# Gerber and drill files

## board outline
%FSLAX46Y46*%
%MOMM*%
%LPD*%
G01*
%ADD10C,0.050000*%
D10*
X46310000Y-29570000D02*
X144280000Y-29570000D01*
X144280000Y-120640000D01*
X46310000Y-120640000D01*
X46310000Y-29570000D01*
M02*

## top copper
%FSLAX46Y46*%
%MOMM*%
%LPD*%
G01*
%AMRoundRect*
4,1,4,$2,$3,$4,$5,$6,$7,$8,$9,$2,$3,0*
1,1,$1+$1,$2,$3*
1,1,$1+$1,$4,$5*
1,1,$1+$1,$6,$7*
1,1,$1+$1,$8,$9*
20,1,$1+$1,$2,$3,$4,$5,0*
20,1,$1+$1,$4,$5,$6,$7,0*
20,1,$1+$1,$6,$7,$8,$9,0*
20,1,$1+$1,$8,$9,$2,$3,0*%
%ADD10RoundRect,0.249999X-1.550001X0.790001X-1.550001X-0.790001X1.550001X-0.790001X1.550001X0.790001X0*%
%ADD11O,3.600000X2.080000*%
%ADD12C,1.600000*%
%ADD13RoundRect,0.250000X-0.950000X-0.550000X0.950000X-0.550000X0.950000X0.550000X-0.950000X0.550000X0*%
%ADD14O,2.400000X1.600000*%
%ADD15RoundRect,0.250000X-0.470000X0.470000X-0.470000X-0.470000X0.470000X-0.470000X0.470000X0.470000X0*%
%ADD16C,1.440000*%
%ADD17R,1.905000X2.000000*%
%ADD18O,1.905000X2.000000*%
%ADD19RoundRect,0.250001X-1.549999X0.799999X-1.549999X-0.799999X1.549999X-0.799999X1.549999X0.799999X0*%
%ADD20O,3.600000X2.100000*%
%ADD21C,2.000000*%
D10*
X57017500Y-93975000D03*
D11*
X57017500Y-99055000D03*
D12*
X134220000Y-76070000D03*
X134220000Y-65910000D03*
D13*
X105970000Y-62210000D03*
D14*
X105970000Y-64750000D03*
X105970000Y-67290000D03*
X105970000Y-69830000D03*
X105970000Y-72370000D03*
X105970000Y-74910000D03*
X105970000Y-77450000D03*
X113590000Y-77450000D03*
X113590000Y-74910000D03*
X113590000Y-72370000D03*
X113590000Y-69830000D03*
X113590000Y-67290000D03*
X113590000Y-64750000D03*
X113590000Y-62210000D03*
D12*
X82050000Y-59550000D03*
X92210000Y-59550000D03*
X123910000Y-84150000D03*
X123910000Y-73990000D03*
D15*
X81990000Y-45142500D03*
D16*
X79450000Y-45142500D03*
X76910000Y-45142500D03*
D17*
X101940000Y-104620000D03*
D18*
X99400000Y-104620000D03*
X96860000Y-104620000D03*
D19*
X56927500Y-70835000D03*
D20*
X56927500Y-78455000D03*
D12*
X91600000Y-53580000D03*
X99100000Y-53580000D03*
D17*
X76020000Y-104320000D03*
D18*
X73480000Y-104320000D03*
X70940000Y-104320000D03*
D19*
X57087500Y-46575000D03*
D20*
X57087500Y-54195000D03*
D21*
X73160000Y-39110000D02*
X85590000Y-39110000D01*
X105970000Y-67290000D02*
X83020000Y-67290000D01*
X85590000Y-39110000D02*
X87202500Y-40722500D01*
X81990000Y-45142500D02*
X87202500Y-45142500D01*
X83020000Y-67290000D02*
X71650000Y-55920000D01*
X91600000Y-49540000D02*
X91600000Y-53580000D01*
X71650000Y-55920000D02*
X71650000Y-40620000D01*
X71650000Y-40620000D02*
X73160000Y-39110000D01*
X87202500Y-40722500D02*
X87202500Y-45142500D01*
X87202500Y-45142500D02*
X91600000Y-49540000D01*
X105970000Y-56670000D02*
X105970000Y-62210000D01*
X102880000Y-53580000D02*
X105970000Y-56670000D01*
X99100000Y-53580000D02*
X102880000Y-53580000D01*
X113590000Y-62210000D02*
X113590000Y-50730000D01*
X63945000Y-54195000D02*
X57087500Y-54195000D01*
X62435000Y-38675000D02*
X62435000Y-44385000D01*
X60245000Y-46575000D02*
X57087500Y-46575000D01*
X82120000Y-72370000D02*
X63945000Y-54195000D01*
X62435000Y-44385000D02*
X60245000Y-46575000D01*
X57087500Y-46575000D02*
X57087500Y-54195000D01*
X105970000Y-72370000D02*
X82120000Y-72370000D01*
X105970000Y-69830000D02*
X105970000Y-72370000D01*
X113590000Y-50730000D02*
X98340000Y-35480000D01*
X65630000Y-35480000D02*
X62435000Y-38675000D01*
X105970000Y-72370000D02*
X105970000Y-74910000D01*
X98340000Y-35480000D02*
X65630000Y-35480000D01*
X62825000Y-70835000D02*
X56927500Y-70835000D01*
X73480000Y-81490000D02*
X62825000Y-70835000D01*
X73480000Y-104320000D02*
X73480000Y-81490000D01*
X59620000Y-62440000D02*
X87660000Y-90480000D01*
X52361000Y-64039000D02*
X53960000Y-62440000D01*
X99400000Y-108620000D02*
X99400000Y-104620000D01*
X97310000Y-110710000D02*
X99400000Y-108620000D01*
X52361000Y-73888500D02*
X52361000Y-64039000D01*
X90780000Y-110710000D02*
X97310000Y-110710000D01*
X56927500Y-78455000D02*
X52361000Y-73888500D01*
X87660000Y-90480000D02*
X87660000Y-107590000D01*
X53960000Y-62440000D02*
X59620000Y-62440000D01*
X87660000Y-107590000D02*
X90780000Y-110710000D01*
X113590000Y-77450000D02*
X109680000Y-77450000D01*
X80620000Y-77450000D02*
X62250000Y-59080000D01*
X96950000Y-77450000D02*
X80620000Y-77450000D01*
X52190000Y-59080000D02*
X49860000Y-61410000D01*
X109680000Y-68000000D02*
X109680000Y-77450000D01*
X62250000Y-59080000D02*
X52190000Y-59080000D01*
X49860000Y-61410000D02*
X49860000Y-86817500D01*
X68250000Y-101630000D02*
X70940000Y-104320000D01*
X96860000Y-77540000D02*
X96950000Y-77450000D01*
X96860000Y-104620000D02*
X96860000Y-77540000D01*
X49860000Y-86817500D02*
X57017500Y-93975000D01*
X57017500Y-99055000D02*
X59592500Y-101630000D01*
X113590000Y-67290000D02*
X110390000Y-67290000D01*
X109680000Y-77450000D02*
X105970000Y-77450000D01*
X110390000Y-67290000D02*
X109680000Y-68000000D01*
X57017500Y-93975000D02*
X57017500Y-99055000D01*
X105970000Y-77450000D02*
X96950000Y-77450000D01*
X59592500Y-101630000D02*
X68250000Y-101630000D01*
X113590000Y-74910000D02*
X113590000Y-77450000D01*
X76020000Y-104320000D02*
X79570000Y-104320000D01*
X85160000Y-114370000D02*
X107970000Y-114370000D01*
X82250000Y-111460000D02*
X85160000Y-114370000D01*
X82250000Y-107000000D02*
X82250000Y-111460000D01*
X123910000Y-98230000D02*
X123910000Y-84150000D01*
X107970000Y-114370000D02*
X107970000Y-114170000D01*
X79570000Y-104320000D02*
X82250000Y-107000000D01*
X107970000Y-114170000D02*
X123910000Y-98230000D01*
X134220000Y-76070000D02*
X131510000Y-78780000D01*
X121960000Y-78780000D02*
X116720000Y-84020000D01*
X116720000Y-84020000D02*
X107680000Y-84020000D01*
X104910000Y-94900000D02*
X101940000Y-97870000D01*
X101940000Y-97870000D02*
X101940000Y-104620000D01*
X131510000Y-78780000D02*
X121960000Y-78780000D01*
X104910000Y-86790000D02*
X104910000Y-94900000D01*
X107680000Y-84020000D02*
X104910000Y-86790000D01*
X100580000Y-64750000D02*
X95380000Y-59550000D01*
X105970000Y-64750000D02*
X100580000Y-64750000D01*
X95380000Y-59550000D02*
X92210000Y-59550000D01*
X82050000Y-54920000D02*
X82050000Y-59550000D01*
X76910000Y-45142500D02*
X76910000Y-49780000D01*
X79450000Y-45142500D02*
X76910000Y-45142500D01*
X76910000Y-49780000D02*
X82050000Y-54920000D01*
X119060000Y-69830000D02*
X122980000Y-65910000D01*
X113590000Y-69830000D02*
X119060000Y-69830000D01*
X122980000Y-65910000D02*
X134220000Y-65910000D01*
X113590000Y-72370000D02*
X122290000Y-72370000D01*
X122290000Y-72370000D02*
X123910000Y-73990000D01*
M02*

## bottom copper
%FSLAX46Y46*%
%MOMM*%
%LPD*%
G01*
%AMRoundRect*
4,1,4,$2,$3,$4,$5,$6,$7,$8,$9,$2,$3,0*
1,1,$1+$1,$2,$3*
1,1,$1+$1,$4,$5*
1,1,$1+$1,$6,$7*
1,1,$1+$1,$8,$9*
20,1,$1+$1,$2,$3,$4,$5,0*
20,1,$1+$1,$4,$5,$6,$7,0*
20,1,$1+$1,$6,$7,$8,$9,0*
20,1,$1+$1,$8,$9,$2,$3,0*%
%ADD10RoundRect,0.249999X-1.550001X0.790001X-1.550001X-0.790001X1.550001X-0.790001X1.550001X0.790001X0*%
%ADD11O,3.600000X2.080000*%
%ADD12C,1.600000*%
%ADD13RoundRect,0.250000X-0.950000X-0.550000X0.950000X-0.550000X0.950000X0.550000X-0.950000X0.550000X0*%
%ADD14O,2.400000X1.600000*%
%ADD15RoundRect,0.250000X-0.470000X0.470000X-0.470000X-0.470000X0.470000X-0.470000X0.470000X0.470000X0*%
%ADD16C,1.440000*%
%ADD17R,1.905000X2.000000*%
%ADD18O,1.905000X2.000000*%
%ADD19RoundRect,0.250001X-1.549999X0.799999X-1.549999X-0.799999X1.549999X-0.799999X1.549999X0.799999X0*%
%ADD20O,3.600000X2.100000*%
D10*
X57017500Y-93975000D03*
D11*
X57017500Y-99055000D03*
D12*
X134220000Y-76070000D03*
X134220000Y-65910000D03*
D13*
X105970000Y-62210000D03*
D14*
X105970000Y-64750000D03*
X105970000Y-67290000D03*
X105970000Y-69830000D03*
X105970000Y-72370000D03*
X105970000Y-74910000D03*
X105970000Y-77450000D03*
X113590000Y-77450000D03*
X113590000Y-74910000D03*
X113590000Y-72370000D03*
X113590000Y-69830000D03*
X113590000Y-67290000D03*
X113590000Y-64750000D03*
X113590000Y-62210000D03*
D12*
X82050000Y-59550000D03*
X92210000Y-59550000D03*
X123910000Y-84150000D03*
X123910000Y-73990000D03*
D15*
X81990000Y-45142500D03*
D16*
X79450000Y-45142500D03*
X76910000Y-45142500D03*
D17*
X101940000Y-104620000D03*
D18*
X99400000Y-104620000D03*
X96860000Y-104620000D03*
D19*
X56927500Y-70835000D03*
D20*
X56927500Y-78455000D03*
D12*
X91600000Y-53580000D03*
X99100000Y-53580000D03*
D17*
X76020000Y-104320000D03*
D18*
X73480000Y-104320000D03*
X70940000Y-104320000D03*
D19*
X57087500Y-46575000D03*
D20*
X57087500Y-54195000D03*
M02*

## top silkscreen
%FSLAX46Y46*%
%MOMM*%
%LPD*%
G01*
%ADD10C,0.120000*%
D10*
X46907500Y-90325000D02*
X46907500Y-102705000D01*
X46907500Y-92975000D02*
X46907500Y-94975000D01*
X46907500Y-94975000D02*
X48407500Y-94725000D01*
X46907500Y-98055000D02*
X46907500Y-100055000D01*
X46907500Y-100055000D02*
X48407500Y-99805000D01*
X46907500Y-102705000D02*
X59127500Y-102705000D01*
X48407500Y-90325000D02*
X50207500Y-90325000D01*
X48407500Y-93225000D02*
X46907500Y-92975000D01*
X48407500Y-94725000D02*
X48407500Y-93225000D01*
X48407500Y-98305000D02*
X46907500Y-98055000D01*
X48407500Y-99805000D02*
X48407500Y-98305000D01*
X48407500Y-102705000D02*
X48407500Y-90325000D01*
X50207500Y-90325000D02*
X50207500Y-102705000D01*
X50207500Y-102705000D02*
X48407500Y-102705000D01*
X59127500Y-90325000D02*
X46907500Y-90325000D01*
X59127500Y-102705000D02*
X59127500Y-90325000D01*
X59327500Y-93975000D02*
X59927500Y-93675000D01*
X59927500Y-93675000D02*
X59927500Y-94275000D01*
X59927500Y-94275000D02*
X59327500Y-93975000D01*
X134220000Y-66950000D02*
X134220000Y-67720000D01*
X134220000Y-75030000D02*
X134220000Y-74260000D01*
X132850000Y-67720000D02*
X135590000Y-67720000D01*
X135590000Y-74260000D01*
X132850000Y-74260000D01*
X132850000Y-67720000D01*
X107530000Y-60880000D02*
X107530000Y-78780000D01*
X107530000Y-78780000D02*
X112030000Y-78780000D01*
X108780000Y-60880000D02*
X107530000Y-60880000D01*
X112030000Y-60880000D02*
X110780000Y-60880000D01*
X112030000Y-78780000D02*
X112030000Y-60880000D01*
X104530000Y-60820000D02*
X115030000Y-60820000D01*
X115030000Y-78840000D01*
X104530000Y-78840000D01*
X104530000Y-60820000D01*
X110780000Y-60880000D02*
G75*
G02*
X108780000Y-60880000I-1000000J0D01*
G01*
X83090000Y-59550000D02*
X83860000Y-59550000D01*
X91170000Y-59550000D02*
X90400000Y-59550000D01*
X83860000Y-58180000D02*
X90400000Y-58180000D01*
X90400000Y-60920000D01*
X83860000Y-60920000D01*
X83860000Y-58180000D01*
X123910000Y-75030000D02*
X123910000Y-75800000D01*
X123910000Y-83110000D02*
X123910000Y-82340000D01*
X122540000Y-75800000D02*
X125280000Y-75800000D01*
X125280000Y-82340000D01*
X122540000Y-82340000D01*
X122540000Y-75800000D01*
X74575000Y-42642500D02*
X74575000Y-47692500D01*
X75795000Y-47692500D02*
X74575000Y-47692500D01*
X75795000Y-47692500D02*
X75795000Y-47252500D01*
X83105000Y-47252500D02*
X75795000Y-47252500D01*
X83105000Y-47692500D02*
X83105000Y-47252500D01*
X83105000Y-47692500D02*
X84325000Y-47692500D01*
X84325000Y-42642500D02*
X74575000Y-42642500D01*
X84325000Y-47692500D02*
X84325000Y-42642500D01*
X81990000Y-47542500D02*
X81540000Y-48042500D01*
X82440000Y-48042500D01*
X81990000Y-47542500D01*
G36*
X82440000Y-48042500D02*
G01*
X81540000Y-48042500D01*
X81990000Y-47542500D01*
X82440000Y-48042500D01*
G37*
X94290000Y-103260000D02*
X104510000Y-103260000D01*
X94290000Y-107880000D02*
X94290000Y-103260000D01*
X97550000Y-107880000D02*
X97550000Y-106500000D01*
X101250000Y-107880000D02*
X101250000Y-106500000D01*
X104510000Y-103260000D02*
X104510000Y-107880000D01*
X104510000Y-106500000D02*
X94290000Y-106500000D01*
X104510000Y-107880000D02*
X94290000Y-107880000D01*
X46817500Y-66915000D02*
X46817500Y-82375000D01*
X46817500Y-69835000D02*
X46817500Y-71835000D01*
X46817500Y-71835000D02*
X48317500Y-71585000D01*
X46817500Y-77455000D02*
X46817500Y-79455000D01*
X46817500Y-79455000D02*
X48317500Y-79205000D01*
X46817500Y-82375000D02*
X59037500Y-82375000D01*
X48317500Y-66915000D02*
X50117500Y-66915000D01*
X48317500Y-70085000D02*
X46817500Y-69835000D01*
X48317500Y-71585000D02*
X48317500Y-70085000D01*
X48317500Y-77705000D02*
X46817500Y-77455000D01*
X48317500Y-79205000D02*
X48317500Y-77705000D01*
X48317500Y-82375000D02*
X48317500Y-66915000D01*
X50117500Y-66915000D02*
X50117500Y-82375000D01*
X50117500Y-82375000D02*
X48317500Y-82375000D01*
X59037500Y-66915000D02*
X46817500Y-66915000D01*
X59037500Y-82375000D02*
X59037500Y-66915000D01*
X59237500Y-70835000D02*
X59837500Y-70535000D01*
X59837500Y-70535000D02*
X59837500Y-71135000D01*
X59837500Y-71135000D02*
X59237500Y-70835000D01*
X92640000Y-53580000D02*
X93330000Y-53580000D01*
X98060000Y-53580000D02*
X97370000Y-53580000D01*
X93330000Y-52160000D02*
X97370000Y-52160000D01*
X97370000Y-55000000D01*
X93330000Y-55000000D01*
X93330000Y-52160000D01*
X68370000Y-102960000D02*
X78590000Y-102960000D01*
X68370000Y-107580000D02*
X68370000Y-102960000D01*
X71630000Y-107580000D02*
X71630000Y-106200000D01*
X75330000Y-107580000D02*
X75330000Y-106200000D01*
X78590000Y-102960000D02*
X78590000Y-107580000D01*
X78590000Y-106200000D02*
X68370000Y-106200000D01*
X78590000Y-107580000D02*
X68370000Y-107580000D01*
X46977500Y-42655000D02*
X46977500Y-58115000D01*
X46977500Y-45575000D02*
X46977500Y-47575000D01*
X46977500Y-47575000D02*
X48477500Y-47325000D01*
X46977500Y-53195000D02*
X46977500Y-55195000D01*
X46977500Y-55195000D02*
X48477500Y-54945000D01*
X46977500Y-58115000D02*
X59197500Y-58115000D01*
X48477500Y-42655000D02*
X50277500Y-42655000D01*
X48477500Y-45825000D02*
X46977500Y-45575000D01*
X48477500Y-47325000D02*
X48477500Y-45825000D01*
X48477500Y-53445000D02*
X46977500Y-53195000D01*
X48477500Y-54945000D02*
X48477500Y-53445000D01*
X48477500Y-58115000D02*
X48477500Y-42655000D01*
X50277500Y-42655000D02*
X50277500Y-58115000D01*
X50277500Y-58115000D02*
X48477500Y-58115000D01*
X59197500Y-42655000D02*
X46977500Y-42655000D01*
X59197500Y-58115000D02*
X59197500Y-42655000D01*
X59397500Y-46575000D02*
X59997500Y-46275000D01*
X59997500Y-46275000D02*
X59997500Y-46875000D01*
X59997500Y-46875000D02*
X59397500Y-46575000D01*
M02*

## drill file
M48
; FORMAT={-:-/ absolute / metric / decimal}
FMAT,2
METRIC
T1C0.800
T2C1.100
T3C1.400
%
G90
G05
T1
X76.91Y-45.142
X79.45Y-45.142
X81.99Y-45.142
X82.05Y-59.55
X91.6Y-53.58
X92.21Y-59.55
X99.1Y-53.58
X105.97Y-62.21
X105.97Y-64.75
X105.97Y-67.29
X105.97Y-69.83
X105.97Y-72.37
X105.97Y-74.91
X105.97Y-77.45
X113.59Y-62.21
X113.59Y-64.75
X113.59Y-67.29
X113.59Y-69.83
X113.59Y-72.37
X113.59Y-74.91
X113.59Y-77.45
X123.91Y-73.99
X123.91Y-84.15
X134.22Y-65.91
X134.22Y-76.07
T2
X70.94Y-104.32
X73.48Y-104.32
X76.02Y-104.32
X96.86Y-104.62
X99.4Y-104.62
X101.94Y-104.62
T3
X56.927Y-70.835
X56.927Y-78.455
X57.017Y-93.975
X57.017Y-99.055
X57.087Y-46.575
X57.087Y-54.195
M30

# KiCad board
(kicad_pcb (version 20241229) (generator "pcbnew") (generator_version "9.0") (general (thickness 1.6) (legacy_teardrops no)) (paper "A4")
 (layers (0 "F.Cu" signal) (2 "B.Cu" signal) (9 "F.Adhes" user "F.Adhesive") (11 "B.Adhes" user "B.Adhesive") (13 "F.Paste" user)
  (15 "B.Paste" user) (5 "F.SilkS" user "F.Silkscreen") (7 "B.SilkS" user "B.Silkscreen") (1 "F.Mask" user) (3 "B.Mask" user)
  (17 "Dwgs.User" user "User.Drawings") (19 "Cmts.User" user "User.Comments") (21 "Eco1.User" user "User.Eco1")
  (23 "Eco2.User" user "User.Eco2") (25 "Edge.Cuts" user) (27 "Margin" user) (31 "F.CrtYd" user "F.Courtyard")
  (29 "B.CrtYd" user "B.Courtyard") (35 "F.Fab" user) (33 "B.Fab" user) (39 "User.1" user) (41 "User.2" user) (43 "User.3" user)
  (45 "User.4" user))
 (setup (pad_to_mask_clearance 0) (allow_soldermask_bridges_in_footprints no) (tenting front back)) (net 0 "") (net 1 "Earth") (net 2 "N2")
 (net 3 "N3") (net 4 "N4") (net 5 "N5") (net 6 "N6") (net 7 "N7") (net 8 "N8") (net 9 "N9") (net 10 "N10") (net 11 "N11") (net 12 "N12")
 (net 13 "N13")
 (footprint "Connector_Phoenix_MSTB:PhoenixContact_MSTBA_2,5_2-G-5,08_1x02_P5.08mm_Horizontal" (layer "F.Cu") (at 57.0175 93.975 -90)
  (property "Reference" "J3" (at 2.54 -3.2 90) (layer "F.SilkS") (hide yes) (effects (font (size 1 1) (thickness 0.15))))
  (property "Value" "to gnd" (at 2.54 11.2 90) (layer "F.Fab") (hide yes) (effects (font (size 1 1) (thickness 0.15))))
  (fp_line (start -3.65 10.11) (end 8.73 10.11) (stroke (width 0.12) (type solid)) (layer "F.SilkS"))
  (fp_line (start -1 10.11) (end 1 10.11) (stroke (width 0.12) (type solid)) (layer "F.SilkS"))
  (fp_line (start 1 10.11) (end 0.75 8.61) (stroke (width 0.12) (type solid)) (layer "F.SilkS"))
  (fp_line (start 4.08 10.11) (end 6.08 10.11) (stroke (width 0.12) (type solid)) (layer "F.SilkS"))
  (fp_line (start 6.08 10.11) (end 5.83 8.61) (stroke (width 0.12) (type solid)) (layer "F.SilkS"))
  (fp_line (start 8.73 10.11) (end 8.73 -2.11) (stroke (width 0.12) (type solid)) (layer "F.SilkS"))
  (fp_line (start -3.65 8.61) (end -3.65 6.81) (stroke (width 0.12) (type solid)) (layer "F.SilkS"))
  (fp_line (start -0.75 8.61) (end -1 10.11) (stroke (width 0.12) (type solid)) (layer "F.SilkS"))
  (fp_line (start 0.75 8.61) (end -0.75 8.61) (stroke (width 0.12) (type solid)) (layer "F.SilkS"))
  (fp_line (start 4.33 8.61) (end 4.08 10.11) (stroke (width 0.12) (type solid)) (layer "F.SilkS"))
  (fp_line (start 5.83 8.61) (end 4.33 8.61) (stroke (width 0.12) (type solid)) (layer "F.SilkS"))
  (fp_line (start 8.73 8.61) (end -3.65 8.61) (stroke (width 0.12) (type solid)) (layer "F.SilkS"))
  (fp_line (start -3.65 6.81) (end 8.73 6.81) (stroke (width 0.12) (type solid)) (layer "F.SilkS"))
  (fp_line (start 8.73 6.81) (end 8.73 8.61) (stroke (width 0.12) (type solid)) (layer "F.SilkS"))
  (fp_line (start -3.65 -2.11) (end -3.65 10.11) (stroke (width 0.12) (type solid)) (layer "F.SilkS"))
  (fp_line (start 8.73 -2.11) (end -3.65 -2.11) (stroke (width 0.12) (type solid)) (layer "F.SilkS"))
  (fp_line (start 0 -2.31) (end -0.3 -2.91) (stroke (width 0.12) (type solid)) (layer "F.SilkS"))
  (fp_line (start -0.3 -2.91) (end 0.3 -2.91) (stroke (width 0.12) (type solid)) (layer "F.SilkS"))
  (fp_line (start 0.3 -2.91) (end 0 -2.31) (stroke (width 0.12) (type solid)) (layer "F.SilkS"))
  (pad "1" thru_hole roundrect (at 0 0 270) (size 2.08 3.6) (drill 1.4) (layers "*.Cu" "*.Mask") (remove_unused_layers no)
   (roundrect_rratio 0.120192) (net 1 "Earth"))
  (pad "2" thru_hole oval (at 5.08 0 270) (size 2.08 3.6) (drill 1.4) (layers "*.Cu" "*.Mask") (remove_unused_layers no) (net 1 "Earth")))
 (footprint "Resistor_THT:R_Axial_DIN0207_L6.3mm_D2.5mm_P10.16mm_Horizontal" (layer "F.Cu") (at 134.22 76.07 90)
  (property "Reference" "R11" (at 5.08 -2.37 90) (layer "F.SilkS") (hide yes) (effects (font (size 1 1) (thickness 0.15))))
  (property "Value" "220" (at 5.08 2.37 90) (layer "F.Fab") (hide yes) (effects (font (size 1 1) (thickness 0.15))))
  (fp_line (start 9.12 0) (end 8.35 0) (stroke (width 0.12) (type solid)) (layer "F.SilkS"))
  (fp_line (start 1.04 0) (end 1.81 0) (stroke (width 0.12) (type solid)) (layer "F.SilkS"))
  (fp_rect (start 1.81 -1.37) (end 8.35 1.37) (stroke (width 0.12) (type solid)) (fill no) (layer "F.SilkS"))
  (pad "1" thru_hole circle (at 0 0 90) (size 1.6 1.6) (drill 0.8) (layers "*.Cu" "*.Mask") (remove_unused_layers no) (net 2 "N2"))
  (pad "2" thru_hole circle (at 10.16 0 90) (size 1.6 1.6) (drill 0.8) (layers "*.Cu" "*.Mask") (remove_unused_layers no) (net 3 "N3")))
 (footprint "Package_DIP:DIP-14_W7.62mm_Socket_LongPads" (layer "F.Cu") (at 105.97 62.21)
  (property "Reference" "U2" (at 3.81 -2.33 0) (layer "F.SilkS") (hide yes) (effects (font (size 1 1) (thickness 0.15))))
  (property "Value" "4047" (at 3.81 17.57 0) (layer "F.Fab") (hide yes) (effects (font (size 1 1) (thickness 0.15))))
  (fp_line (start 1.56 -1.33) (end 1.56 16.57) (stroke (width 0.12) (type solid)) (layer "F.SilkS"))
  (fp_line (start 1.56 16.57) (end 6.06 16.57) (stroke (width 0.12) (type solid)) (layer "F.SilkS"))
  (fp_line (start 2.81 -1.33) (end 1.56 -1.33) (stroke (width 0.12) (type solid)) (layer "F.SilkS"))
  (fp_line (start 6.06 -1.33) (end 4.81 -1.33) (stroke (width 0.12) (type solid)) (layer "F.SilkS"))
  (fp_line (start 6.06 16.57) (end 6.06 -1.33) (stroke (width 0.12) (type solid)) (layer "F.SilkS"))
  (fp_rect (start -1.44 -1.39) (end 9.06 16.63) (stroke (width 0.12) (type solid)) (fill no) (layer "F.SilkS"))
  (fp_arc (start 4.81 -1.33) (mid 3.81 -0.33) (end 2.81 -1.33) (stroke (width 0.12) (type solid)) (layer "F.SilkS"))
  (pad "1" thru_hole roundrect (at 0 0) (size 2.4 1.6) (drill 0.8) (layers "*.Cu" "*.Mask") (remove_unused_layers no)
   (roundrect_rratio 0.15625) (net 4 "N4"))
  (pad "2" thru_hole oval (at 0 2.54) (size 2.4 1.6) (drill 0.8) (layers "*.Cu" "*.Mask") (remove_unused_layers no) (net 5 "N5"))
  (pad "3" thru_hole oval (at 0 5.08) (size 2.4 1.6) (drill 0.8) (layers "*.Cu" "*.Mask") (remove_unused_layers no) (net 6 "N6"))
  (pad "4" thru_hole oval (at 0 7.62) (size 2.4 1.6) (drill 0.8) (layers "*.Cu" "*.Mask") (remove_unused_layers no) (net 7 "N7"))
  (pad "5" thru_hole oval (at 0 10.16) (size 2.4 1.6) (drill 0.8) (layers "*.Cu" "*.Mask") (remove_unused_layers no) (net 7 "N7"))
  (pad "6" thru_hole oval (at 0 12.7) (size 2.4 1.6) (drill 0.8) (layers "*.Cu" "*.Mask") (remove_unused_layers no) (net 7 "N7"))
  (pad "7" thru_hole oval (at 0 15.24) (size 2.4 1.6) (drill 0.8) (layers "*.Cu" "*.Mask") (remove_unused_layers no) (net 1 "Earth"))
  (pad "8" thru_hole oval (at 7.62 15.24) (size 2.4 1.6) (drill 0.8) (layers "*.Cu" "*.Mask") (remove_unused_layers no) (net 1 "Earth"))
  (pad "9" thru_hole oval (at 7.62 12.7) (size 2.4 1.6) (drill 0.8) (layers "*.Cu" "*.Mask") (remove_unused_layers no) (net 1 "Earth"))
  (pad "10" thru_hole oval (at 7.62 10.16) (size 2.4 1.6) (drill 0.8) (layers "*.Cu" "*.Mask") (remove_unused_layers no) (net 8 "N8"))
  (pad "11" thru_hole oval (at 7.62 7.62) (size 2.4 1.6) (drill 0.8) (layers "*.Cu" "*.Mask") (remove_unused_layers no) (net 3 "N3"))
  (pad "12" thru_hole oval (at 7.62 5.08) (size 2.4 1.6) (drill 0.8) (layers "*.Cu" "*.Mask") (remove_unused_layers no) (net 1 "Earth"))
  (pad "13" thru_hole oval (at 7.62 2.54) (size 2.4 1.6) (drill 0.8) (layers "*.Cu" "*.Mask") (remove_unused_layers no) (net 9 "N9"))
  (pad "14" thru_hole oval (at 7.62 0) (size 2.4 1.6) (drill 0.8) (layers "*.Cu" "*.Mask") (remove_unused_layers no) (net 7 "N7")))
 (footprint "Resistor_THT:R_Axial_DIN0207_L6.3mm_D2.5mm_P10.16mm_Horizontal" (layer "F.Cu") (at 82.05 59.55)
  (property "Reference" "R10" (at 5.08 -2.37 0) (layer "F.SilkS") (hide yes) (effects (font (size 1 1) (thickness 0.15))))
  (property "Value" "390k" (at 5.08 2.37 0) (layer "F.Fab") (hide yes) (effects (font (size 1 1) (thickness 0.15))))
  (fp_line (start 1.04 0) (end 1.81 0) (stroke (width 0.12) (type solid)) (layer "F.SilkS"))
  (fp_line (start 9.12 0) (end 8.35 0) (stroke (width 0.12) (type solid)) (layer "F.SilkS"))
  (fp_rect (start 1.81 -1.37) (end 8.35 1.37) (stroke (width 0.12) (type solid)) (fill no) (layer "F.SilkS"))
  (pad "1" thru_hole circle (at 0 0) (size 1.6 1.6) (drill 0.8) (layers "*.Cu" "*.Mask") (remove_unused_layers no) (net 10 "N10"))
  (pad "2" thru_hole circle (at 10.16 0) (size 1.6 1.6) (drill 0.8) (layers "*.Cu" "*.Mask") (remove_unused_layers no) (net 5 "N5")))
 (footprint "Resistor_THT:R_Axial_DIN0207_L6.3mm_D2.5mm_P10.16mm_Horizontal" (layer "F.Cu") (at 123.91 84.15 90)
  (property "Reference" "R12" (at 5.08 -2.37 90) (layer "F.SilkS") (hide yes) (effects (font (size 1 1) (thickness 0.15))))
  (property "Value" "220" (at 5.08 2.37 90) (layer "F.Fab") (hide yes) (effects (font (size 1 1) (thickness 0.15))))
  (fp_line (start 9.12 0) (end 8.35 0) (stroke (width 0.12) (type solid)) (layer "F.SilkS"))
  (fp_line (start 1.04 0) (end 1.81 0) (stroke (width 0.12) (type solid)) (layer "F.SilkS"))
  (fp_rect (start 1.81 -1.37) (end 8.35 1.37) (stroke (width 0.12) (type solid)) (fill no) (layer "F.SilkS"))
  (pad "1" thru_hole circle (at 0 0 90) (size 1.6 1.6) (drill 0.8) (layers "*.Cu" "*.Mask") (remove_unused_layers no) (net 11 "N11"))
  (pad "2" thru_hole circle (at 10.16 0 90) (size 1.6 1.6) (drill 0.8) (layers "*.Cu" "*.Mask") (remove_unused_layers no) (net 8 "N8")))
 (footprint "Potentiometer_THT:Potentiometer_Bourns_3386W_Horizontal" (layer "F.Cu") (at 81.99 45.1425 180)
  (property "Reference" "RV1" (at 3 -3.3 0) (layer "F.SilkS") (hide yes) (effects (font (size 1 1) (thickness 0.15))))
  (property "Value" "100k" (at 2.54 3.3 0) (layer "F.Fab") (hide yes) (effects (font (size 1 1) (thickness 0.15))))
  (fp_line (start 7.415 2.5) (end 7.415 -2.55) (stroke (width 0.12) (type default)) (layer "F.SilkS"))
  (fp_line (start 6.195 -2.55) (end 7.415 -2.55) (stroke (width 0.12) (type default)) (layer "F.SilkS"))
  (fp_line (start 6.195 -2.55) (end 6.195 -2.11) (stroke (width 0.12) (type default)) (layer "F.SilkS"))
  (fp_line (start -1.115 -2.11) (end 6.195 -2.11) (stroke (width 0.12) (type default)) (layer "F.SilkS"))
  (fp_line (start -1.115 -2.55) (end -1.115 -2.11) (stroke (width 0.12) (type default)) (layer "F.SilkS"))
  (fp_line (start -1.115 -2.55) (end -2.335 -2.55) (stroke (width 0.12) (type default)) (layer "F.SilkS"))
  (fp_line (start -2.335 2.5) (end 7.415 2.5) (stroke (width 0.12) (type default)) (layer "F.SilkS"))
  (fp_line (start -2.335 -2.55) (end -2.335 2.5) (stroke (width 0.12) (type default)) (layer "F.SilkS"))
  (fp_poly (pts (xy 0 -2.4) (xy 0.45 -2.9) (xy -0.45 -2.9)) (stroke (width 0.12) (type solid)) (fill yes) (layer "F.SilkS"))
  (pad "1" thru_hole roundrect (at 0 0 270) (size 1.44 1.44) (drill 0.8) (layers "*.Cu" "*.Mask") (remove_unused_layers no)
   (roundrect_rratio 0.1736111111) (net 6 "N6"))
  (pad "2" thru_hole circle (at 2.54 0 270) (size 1.44 1.44) (drill 0.8) (layers "*.Cu" "*.Mask") (remove_unused_layers no) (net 10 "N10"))
  (pad "3" thru_hole circle (at 5.08 0 270) (size 1.44 1.44) (drill 0.8) (layers "*.Cu" "*.Mask") (remove_unused_layers no) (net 10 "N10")))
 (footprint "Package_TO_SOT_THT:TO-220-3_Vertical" (layer "F.Cu") (at 101.94 104.62 180)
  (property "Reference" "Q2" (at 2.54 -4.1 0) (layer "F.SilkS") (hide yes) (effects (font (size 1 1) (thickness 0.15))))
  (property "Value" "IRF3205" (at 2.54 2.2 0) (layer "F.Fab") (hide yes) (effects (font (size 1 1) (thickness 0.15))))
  (fp_line (start 7.65 1.36) (end -2.57 1.36) (stroke (width 0.12) (type solid)) (layer "F.SilkS"))
  (fp_line (start 7.65 -3.26) (end 7.65 1.36) (stroke (width 0.12) (type solid)) (layer "F.SilkS"))
  (fp_line (start 4.39 -3.26) (end 4.39 -1.88) (stroke (width 0.12) (type solid)) (layer "F.SilkS"))
  (fp_line (start 0.69 -3.26) (end 0.69 -1.88) (stroke (width 0.12) (type solid)) (layer "F.SilkS"))
  (fp_line (start -2.57 1.36) (end -2.57 -3.26) (stroke (width 0.12) (type solid)) (layer "F.SilkS"))
  (fp_line (start -2.57 -1.88) (end 7.65 -1.88) (stroke (width 0.12) (type solid)) (layer "F.SilkS"))
  (fp_line (start -2.57 -3.26) (end 7.65 -3.26) (stroke (width 0.12) (type solid)) (layer "F.SilkS"))
  (pad "1" thru_hole rect (at 0 0 180) (size 1.905 2) (drill 1.1) (layers "*.Cu" "*.Mask") (remove_unused_layers no) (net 2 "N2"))
  (pad "2" thru_hole oval (at 2.54 0 180) (size 1.905 2) (drill 1.1) (layers "*.Cu" "*.Mask") (remove_unused_layers no) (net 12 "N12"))
  (pad "3" thru_hole oval (at 5.08 0 180) (size 1.905 2) (drill 1.1) (layers "*.Cu" "*.Mask") (remove_unused_layers no) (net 1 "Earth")))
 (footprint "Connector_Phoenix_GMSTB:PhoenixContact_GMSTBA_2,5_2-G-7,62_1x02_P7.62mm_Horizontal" (layer "F.Cu") (at 56.9275 70.835 -90)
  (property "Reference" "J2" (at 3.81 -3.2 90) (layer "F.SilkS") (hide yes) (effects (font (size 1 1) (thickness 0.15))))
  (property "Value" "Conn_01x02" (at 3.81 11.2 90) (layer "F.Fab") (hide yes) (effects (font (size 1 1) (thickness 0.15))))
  (fp_line (start -3.92 10.11) (end 11.54 10.11) (stroke (width 0.12) (type solid)) (layer "F.SilkS"))
  (fp_line (start -1 10.11) (end 1 10.11) (stroke (width 0.12) (type solid)) (layer "F.SilkS"))
  (fp_line (start 1 10.11) (end 0.75 8.61) (stroke (width 0.12) (type solid)) (layer "F.SilkS"))
  (fp_line (start 6.62 10.11) (end 8.62 10.11) (stroke (width 0.12) (type solid)) (layer "F.SilkS"))
  (fp_line (start 8.62 10.11) (end 8.37 8.61) (stroke (width 0.12) (type solid)) (layer "F.SilkS"))
  (fp_line (start 11.54 10.11) (end 11.54 -2.11) (stroke (width 0.12) (type solid)) (layer "F.SilkS"))
  (fp_line (start -3.92 8.61) (end -3.92 6.81) (stroke (width 0.12) (type solid)) (layer "F.SilkS"))
  (fp_line (start -0.75 8.61) (end -1 10.11) (stroke (width 0.12) (type solid)) (layer "F.SilkS"))
  (fp_line (start 0.75 8.61) (end -0.75 8.61) (stroke (width 0.12) (type solid)) (layer "F.SilkS"))
  (fp_line (start 6.87 8.61) (end 6.62 10.11) (stroke (width 0.12) (type solid)) (layer "F.SilkS"))
  (fp_line (start 8.37 8.61) (end 6.87 8.61) (stroke (width 0.12) (type solid)) (layer "F.SilkS"))
  (fp_line (start 11.54 8.61) (end -3.92 8.61) (stroke (width 0.12) (type solid)) (layer "F.SilkS"))
  (fp_line (start -3.92 6.81) (end 11.54 6.81) (stroke (width 0.12) (type solid)) (layer "F.SilkS"))
  (fp_line (start 11.54 6.81) (end 11.54 8.61) (stroke (width 0.12) (type solid)) (layer "F.SilkS"))
  (fp_line (start -3.92 -2.11) (end -3.92 10.11) (stroke (width 0.12) (type solid)) (layer "F.SilkS"))
  (fp_line (start 11.54 -2.11) (end -3.92 -2.11) (stroke (width 0.12) (type solid)) (layer "F.SilkS"))
  (fp_line (start 0 -2.31) (end -0.3 -2.91) (stroke (width 0.12) (type solid)) (layer "F.SilkS"))
  (fp_line (start -0.3 -2.91) (end 0.3 -2.91) (stroke (width 0.12) (type solid)) (layer "F.SilkS"))
  (fp_line (start 0.3 -2.91) (end 0 -2.31) (stroke (width 0.12) (type solid)) (layer "F.SilkS"))
  (pad "1" thru_hole roundrect (at 0 0 270) (size 2.1 3.6) (drill 1.4) (layers "*.Cu" "*.Mask") (remove_unused_layers no)
   (roundrect_rratio 0.119048) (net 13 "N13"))
  (pad "2" thru_hole oval (at 7.62 0 270) (size 2.1 3.6) (drill 1.4) (layers "*.Cu" "*.Mask") (remove_unused_layers no) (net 12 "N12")))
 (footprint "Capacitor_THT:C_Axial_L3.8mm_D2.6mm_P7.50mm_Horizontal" (layer "F.Cu") (at 91.6 53.58)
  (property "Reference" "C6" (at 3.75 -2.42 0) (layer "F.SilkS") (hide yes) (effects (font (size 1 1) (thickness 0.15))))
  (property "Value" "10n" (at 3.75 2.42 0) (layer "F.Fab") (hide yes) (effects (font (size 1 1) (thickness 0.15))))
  (fp_line (start 1.04 0) (end 1.73 0) (stroke (width 0.12) (type solid)) (layer "F.SilkS"))
  (fp_line (start 6.46 0) (end 5.77 0) (stroke (width 0.12) (type solid)) (layer "F.SilkS"))
  (fp_rect (start 1.73 -1.42) (end 5.77 1.42) (stroke (width 0.12) (type solid)) (fill no) (layer "F.SilkS"))
  (pad "1" thru_hole circle (at 0 0) (size 1.6 1.6) (drill 0.8) (layers "*.Cu" "*.Mask") (remove_unused_layers no) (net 6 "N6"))
  (pad "2" thru_hole circle (at 7.5 0) (size 1.6 1.6) (drill 0.8) (layers "*.Cu" "*.Mask") (remove_unused_layers no) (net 4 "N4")))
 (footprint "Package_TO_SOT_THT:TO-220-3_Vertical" (layer "F.Cu") (at 76.02 104.32 180)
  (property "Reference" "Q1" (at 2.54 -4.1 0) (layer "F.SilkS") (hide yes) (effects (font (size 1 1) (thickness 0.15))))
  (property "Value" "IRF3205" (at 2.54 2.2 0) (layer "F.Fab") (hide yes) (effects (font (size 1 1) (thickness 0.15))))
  (fp_line (start 7.65 1.36) (end -2.57 1.36) (stroke (width 0.12) (type solid)) (layer "F.SilkS"))
  (fp_line (start 7.65 -3.26) (end 7.65 1.36) (stroke (width 0.12) (type solid)) (layer "F.SilkS"))
  (fp_line (start 4.39 -3.26) (end 4.39 -1.88) (stroke (width 0.12) (type solid)) (layer "F.SilkS"))
  (fp_line (start 0.69 -3.26) (end 0.69 -1.88) (stroke (width 0.12) (type solid)) (layer "F.SilkS"))
  (fp_line (start -2.57 1.36) (end -2.57 -3.26) (stroke (width 0.12) (type solid)) (layer "F.SilkS"))
  (fp_line (start -2.57 -1.88) (end 7.65 -1.88) (stroke (width 0.12) (type solid)) (layer "F.SilkS"))
  (fp_line (start -2.57 -3.26) (end 7.65 -3.26) (stroke (width 0.12) (type solid)) (layer "F.SilkS"))
  (pad "1" thru_hole rect (at 0 0 180) (size 1.905 2) (drill 1.1) (layers "*.Cu" "*.Mask") (remove_unused_layers no) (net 11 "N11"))
  (pad "2" thru_hole oval (at 2.54 0 180) (size 1.905 2) (drill 1.1) (layers "*.Cu" "*.Mask") (remove_unused_layers no) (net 13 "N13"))
  (pad "3" thru_hole oval (at 5.08 0 180) (size 1.905 2) (drill 1.1) (layers "*.Cu" "*.Mask") (remove_unused_layers no) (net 1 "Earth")))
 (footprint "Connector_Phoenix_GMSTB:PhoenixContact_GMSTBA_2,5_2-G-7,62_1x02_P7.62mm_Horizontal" (layer "F.Cu") (at 57.0875 46.575 -90)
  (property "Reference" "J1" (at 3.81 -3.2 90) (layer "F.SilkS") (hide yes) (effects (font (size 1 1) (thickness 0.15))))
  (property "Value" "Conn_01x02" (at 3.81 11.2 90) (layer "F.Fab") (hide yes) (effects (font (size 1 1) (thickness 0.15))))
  (fp_line (start -3.92 10.11) (end 11.54 10.11) (stroke (width 0.12) (type solid)) (layer "F.SilkS"))
  (fp_line (start -1 10.11) (end 1 10.11) (stroke (width 0.12) (type solid)) (layer "F.SilkS"))
  (fp_line (start 1 10.11) (end 0.75 8.61) (stroke (width 0.12) (type solid)) (layer "F.SilkS"))
  (fp_line (start 6.62 10.11) (end 8.62 10.11) (stroke (width 0.12) (type solid)) (layer "F.SilkS"))
  (fp_line (start 8.62 10.11) (end 8.37 8.61) (stroke (width 0.12) (type solid)) (layer "F.SilkS"))
  (fp_line (start 11.54 10.11) (end 11.54 -2.11) (stroke (width 0.12) (type solid)) (layer "F.SilkS"))
  (fp_line (start -3.92 8.61) (end -3.92 6.81) (stroke (width 0.12) (type solid)) (layer "F.SilkS"))
  (fp_line (start -0.75 8.61) (end -1 10.11) (stroke (width 0.12) (type solid)) (layer "F.SilkS"))
  (fp_line (start 0.75 8.61) (end -0.75 8.61) (stroke (width 0.12) (type solid)) (layer "F.SilkS"))
  (fp_line (start 6.87 8.61) (end 6.62 10.11) (stroke (width 0.12) (type solid)) (layer "F.SilkS"))
  (fp_line (start 8.37 8.61) (end 6.87 8.61) (stroke (width 0.12) (type solid)) (layer "F.SilkS"))
  (fp_line (start 11.54 8.61) (end -3.92 8.61) (stroke (width 0.12) (type solid)) (layer "F.SilkS"))
  (fp_line (start -3.92 6.81) (end 11.54 6.81) (stroke (width 0.12) (type solid)) (layer "F.SilkS"))
  (fp_line (start 11.54 6.81) (end 11.54 8.61) (stroke (width 0.12) (type solid)) (layer "F.SilkS"))
  (fp_line (start -3.92 -2.11) (end -3.92 10.11) (stroke (width 0.12) (type solid)) (layer "F.SilkS"))
  (fp_line (start 11.54 -2.11) (end -3.92 -2.11) (stroke (width 0.12) (type solid)) (layer "F.SilkS"))
  (fp_line (start 0 -2.31) (end -0.3 -2.91) (stroke (width 0.12) (type solid)) (layer "F.SilkS"))
  (fp_line (start -0.3 -2.91) (end 0.3 -2.91) (stroke (width 0.12) (type solid)) (layer "F.SilkS"))
  (fp_line (start 0.3 -2.91) (end 0 -2.31) (stroke (width 0.12) (type solid)) (layer "F.SilkS"))
  (pad "1" thru_hole roundrect (at 0 0 270) (size 2.1 3.6) (drill 1.4) (layers "*.Cu" "*.Mask") (remove_unused_layers no)
   (roundrect_rratio 0.119048) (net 7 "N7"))
  (pad "2" thru_hole oval (at 7.62 0 270) (size 2.1 3.6) (drill 1.4) (layers "*.Cu" "*.Mask") (remove_unused_layers no) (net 7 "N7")))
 (gr_rect (start 46.31 29.57) (end 144.28 120.64) (stroke (width 0.05) (type default)) (fill no) (layer "Edge.Cuts"))
 (segment (start 73.16 39.11) (end 85.59 39.11) (width 2) (layer "F.Cu") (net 6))
 (segment (start 105.97 67.29) (end 83.02 67.29) (width 2) (layer "F.Cu") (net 6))
 (segment (start 85.59 39.11) (end 87.2025 40.7225) (width 2) (layer "F.Cu") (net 6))
 (segment (start 81.99 45.1425) (end 87.2025 45.1425) (width 2) (layer "F.Cu") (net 6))
 (segment (start 83.02 67.29) (end 71.65 55.92) (width 2) (layer "F.Cu") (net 6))
 (segment (start 91.6 49.54) (end 91.6 53.58) (width 2) (layer "F.Cu") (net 6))
 (segment (start 71.65 55.92) (end 71.65 40.62) (width 2) (layer "F.Cu") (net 6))
 (segment (start 71.65 40.62) (end 73.16 39.11) (width 2) (layer "F.Cu") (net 6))
 (segment (start 87.2025 40.7225) (end 87.2025 45.1425) (width 2) (layer "F.Cu") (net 6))
 (segment (start 87.2025 45.1425) (end 91.6 49.54) (width 2) (layer "F.Cu") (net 6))
 (segment (start 105.97 56.67) (end 105.97 62.21) (width 2) (layer "F.Cu") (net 4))
 (segment (start 102.88 53.58) (end 105.97 56.67) (width 2) (layer "F.Cu") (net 4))
 (segment (start 99.1 53.58) (end 102.88 53.58) (width 2) (layer "F.Cu") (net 4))
 (segment (start 113.59 62.21) (end 113.59 50.73) (width 2) (layer "F.Cu") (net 7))
 (segment (start 63.945 54.195) (end 57.0875 54.195) (width 2) (layer "F.Cu") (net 7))
 (segment (start 62.435 38.675) (end 62.435 44.385) (width 2) (layer "F.Cu") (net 7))
 (segment (start 60.245 46.575) (end 57.0875 46.575) (width 2) (layer "F.Cu") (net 7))
 (segment (start 82.12 72.37) (end 63.945 54.195) (width 2) (layer "F.Cu") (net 7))
 (segment (start 62.435 44.385) (end 60.245 46.575) (width 2) (layer "F.Cu") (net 7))
 (segment (start 57.0875 46.575) (end 57.0875 54.195) (width 2) (layer "F.Cu") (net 7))
 (segment (start 105.97 72.37) (end 82.12 72.37) (width 2) (layer "F.Cu") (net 7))
 (segment (start 105.97 69.83) (end 105.97 72.37) (width 2) (layer "F.Cu") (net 7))
 (segment (start 113.59 50.73) (end 98.34 35.48) (width 2) (layer "F.Cu") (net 7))
 (segment (start 65.63 35.48) (end 62.435 38.675) (width 2) (layer "F.Cu") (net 7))
 (segment (start 105.97 72.37) (end 105.97 74.91) (width 2) (layer "F.Cu") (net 7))
 (segment (start 98.34 35.48) (end 65.63 35.48) (width 2) (layer "F.Cu") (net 7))
 (segment (start 62.825 70.835) (end 56.9275 70.835) (width 2) (layer "F.Cu") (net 13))
 (segment (start 73.48 81.49) (end 62.825 70.835) (width 2) (layer "F.Cu") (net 13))
 (segment (start 73.48 104.32) (end 73.48 81.49) (width 2) (layer "F.Cu") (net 13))
 (segment (start 59.62 62.44) (end 87.66 90.48) (width 2) (layer "F.Cu") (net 12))
 (segment (start 52.361 64.039) (end 53.96 62.44) (width 2) (layer "F.Cu") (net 12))
 (segment (start 99.4 108.62) (end 99.4 104.62) (width 2) (layer "F.Cu") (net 12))
 (segment (start 97.31 110.71) (end 99.4 108.62) (width 2) (layer "F.Cu") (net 12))
 (segment (start 52.361 73.8885) (end 52.361 64.039) (width 2) (layer "F.Cu") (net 12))
 (segment (start 90.78 110.71) (end 97.31 110.71) (width 2) (layer "F.Cu") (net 12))
 (segment (start 56.9275 78.455) (end 52.361 73.8885) (width 2) (layer "F.Cu") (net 12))
 (segment (start 87.66 90.48) (end 87.66 107.59) (width 2) (layer "F.Cu") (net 12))
 (segment (start 53.96 62.44) (end 59.62 62.44) (width 2) (layer "F.Cu") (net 12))
 (segment (start 87.66 107.59) (end 90.78 110.71) (width 2) (layer "F.Cu") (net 12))
 (segment (start 113.59 77.45) (end 109.68 77.45) (width 2) (layer "F.Cu") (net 1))
 (segment (start 80.62 77.45) (end 62.25 59.08) (width 2) (layer "F.Cu") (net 1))
 (segment (start 96.95 77.45) (end 80.62 77.45) (width 2) (layer "F.Cu") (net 1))
 (segment (start 52.19 59.08) (end 49.86 61.41) (width 2) (layer "F.Cu") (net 1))
 (segment (start 109.68 68) (end 109.68 77.45) (width 2) (layer "F.Cu") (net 1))
 (segment (start 62.25 59.08) (end 52.19 59.08) (width 2) (layer "F.Cu") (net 1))
 (segment (start 49.86 61.41) (end 49.86 86.8175) (width 2) (layer "F.Cu") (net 1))
 (segment (start 68.25 101.63) (end 70.94 104.32) (width 2) (layer "F.Cu") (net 1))
 (segment (start 96.86 77.54) (end 96.95 77.45) (width 2) (layer "F.Cu") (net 1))
 (segment (start 96.86 104.62) (end 96.86 77.54) (width 2) (layer "F.Cu") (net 1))
 (segment (start 49.86 86.8175) (end 57.0175 93.975) (width 2) (layer "F.Cu") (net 1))
 (segment (start 57.0175 99.055) (end 59.5925 101.63) (width 2) (layer "F.Cu") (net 1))
 (segment (start 113.59 67.29) (end 110.39 67.29) (width 2) (layer "F.Cu") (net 1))
 (segment (start 109.68 77.45) (end 105.97 77.45) (width 2) (layer "F.Cu") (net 1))
 (segment (start 110.39 67.29) (end 109.68 68) (width 2) (layer "F.Cu") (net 1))
 (segment (start 57.0175 93.975) (end 57.0175 99.055) (width 2) (layer "F.Cu") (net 1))
 (segment (start 105.97 77.45) (end 96.95 77.45) (width 2) (layer "F.Cu") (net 1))
 (segment (start 59.5925 101.63) (end 68.25 101.63) (width 2) (layer "F.Cu") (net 1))
 (segment (start 113.59 74.91) (end 113.59 77.45) (width 2) (layer "F.Cu") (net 1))
 (segment (start 76.02 104.32) (end 79.57 104.32) (width 2) (layer "F.Cu") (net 11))
 (segment (start 85.16 114.37) (end 107.97 114.37) (width 2) (layer "F.Cu") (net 11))
 (segment (start 82.25 111.46) (end 85.16 114.37) (width 2) (layer "F.Cu") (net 11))
 (segment (start 82.25 107) (end 82.25 111.46) (width 2) (layer "F.Cu") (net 11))
 (segment (start 123.91 98.23) (end 123.91 84.15) (width 2) (layer "F.Cu") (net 11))
 (segment (start 107.97 114.37) (end 107.97 114.17) (width 2) (layer "F.Cu") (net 11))
 (segment (start 79.57 104.32) (end 82.25 107) (width 2) (layer "F.Cu") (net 11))
 (segment (start 107.97 114.17) (end 123.91 98.23) (width 2) (layer "F.Cu") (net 11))
 (segment (start 134.22 76.07) (end 131.51 78.78) (width 2) (layer "F.Cu") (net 2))
 (segment (start 121.96 78.78) (end 116.72 84.02) (width 2) (layer "F.Cu") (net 2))
 (segment (start 116.72 84.02) (end 107.68 84.02) (width 2) (layer "F.Cu") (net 2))
 (segment (start 104.91 94.9) (end 101.94 97.87) (width 2) (layer "F.Cu") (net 2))
 (segment (start 101.94 97.87) (end 101.94 104.62) (width 2) (layer "F.Cu") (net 2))
 (segment (start 131.51 78.78) (end 121.96 78.78) (width 2) (layer "F.Cu") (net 2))
 (segment (start 104.91 86.79) (end 104.91 94.9) (width 2) (layer "F.Cu") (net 2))
 (segment (start 107.68 84.02) (end 104.91 86.79) (width 2) (layer "F.Cu") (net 2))
 (segment (start 100.58 64.75) (end 95.38 59.55) (width 2) (layer "F.Cu") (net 5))
 (segment (start 105.97 64.75) (end 100.58 64.75) (width 2) (layer "F.Cu") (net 5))
 (segment (start 95.38 59.55) (end 92.21 59.55) (width 2) (layer "F.Cu") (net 5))
 (segment (start 82.05 54.92) (end 82.05 59.55) (width 2) (layer "F.Cu") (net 10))
 (segment (start 76.91 45.1425) (end 76.91 49.78) (width 2) (layer "F.Cu") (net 10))
 (segment (start 79.45 45.1425) (end 76.91 45.1425) (width 2) (layer "F.Cu") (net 10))
 (segment (start 76.91 49.78) (end 82.05 54.92) (width 2) (layer "F.Cu") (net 10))
 (segment (start 119.06 69.83) (end 122.98 65.91) (width 2) (layer "F.Cu") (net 3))
 (segment (start 113.59 69.83) (end 119.06 69.83) (width 2) (layer "F.Cu") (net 3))
 (segment (start 122.98 65.91) (end 134.22 65.91) (width 2) (layer "F.Cu") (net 3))
 (segment (start 113.59 72.37) (end 122.29 72.37) (width 2) (layer "F.Cu") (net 8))
 (segment (start 122.29 72.37) (end 123.91 73.99) (width 2) (layer "F.Cu") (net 8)))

